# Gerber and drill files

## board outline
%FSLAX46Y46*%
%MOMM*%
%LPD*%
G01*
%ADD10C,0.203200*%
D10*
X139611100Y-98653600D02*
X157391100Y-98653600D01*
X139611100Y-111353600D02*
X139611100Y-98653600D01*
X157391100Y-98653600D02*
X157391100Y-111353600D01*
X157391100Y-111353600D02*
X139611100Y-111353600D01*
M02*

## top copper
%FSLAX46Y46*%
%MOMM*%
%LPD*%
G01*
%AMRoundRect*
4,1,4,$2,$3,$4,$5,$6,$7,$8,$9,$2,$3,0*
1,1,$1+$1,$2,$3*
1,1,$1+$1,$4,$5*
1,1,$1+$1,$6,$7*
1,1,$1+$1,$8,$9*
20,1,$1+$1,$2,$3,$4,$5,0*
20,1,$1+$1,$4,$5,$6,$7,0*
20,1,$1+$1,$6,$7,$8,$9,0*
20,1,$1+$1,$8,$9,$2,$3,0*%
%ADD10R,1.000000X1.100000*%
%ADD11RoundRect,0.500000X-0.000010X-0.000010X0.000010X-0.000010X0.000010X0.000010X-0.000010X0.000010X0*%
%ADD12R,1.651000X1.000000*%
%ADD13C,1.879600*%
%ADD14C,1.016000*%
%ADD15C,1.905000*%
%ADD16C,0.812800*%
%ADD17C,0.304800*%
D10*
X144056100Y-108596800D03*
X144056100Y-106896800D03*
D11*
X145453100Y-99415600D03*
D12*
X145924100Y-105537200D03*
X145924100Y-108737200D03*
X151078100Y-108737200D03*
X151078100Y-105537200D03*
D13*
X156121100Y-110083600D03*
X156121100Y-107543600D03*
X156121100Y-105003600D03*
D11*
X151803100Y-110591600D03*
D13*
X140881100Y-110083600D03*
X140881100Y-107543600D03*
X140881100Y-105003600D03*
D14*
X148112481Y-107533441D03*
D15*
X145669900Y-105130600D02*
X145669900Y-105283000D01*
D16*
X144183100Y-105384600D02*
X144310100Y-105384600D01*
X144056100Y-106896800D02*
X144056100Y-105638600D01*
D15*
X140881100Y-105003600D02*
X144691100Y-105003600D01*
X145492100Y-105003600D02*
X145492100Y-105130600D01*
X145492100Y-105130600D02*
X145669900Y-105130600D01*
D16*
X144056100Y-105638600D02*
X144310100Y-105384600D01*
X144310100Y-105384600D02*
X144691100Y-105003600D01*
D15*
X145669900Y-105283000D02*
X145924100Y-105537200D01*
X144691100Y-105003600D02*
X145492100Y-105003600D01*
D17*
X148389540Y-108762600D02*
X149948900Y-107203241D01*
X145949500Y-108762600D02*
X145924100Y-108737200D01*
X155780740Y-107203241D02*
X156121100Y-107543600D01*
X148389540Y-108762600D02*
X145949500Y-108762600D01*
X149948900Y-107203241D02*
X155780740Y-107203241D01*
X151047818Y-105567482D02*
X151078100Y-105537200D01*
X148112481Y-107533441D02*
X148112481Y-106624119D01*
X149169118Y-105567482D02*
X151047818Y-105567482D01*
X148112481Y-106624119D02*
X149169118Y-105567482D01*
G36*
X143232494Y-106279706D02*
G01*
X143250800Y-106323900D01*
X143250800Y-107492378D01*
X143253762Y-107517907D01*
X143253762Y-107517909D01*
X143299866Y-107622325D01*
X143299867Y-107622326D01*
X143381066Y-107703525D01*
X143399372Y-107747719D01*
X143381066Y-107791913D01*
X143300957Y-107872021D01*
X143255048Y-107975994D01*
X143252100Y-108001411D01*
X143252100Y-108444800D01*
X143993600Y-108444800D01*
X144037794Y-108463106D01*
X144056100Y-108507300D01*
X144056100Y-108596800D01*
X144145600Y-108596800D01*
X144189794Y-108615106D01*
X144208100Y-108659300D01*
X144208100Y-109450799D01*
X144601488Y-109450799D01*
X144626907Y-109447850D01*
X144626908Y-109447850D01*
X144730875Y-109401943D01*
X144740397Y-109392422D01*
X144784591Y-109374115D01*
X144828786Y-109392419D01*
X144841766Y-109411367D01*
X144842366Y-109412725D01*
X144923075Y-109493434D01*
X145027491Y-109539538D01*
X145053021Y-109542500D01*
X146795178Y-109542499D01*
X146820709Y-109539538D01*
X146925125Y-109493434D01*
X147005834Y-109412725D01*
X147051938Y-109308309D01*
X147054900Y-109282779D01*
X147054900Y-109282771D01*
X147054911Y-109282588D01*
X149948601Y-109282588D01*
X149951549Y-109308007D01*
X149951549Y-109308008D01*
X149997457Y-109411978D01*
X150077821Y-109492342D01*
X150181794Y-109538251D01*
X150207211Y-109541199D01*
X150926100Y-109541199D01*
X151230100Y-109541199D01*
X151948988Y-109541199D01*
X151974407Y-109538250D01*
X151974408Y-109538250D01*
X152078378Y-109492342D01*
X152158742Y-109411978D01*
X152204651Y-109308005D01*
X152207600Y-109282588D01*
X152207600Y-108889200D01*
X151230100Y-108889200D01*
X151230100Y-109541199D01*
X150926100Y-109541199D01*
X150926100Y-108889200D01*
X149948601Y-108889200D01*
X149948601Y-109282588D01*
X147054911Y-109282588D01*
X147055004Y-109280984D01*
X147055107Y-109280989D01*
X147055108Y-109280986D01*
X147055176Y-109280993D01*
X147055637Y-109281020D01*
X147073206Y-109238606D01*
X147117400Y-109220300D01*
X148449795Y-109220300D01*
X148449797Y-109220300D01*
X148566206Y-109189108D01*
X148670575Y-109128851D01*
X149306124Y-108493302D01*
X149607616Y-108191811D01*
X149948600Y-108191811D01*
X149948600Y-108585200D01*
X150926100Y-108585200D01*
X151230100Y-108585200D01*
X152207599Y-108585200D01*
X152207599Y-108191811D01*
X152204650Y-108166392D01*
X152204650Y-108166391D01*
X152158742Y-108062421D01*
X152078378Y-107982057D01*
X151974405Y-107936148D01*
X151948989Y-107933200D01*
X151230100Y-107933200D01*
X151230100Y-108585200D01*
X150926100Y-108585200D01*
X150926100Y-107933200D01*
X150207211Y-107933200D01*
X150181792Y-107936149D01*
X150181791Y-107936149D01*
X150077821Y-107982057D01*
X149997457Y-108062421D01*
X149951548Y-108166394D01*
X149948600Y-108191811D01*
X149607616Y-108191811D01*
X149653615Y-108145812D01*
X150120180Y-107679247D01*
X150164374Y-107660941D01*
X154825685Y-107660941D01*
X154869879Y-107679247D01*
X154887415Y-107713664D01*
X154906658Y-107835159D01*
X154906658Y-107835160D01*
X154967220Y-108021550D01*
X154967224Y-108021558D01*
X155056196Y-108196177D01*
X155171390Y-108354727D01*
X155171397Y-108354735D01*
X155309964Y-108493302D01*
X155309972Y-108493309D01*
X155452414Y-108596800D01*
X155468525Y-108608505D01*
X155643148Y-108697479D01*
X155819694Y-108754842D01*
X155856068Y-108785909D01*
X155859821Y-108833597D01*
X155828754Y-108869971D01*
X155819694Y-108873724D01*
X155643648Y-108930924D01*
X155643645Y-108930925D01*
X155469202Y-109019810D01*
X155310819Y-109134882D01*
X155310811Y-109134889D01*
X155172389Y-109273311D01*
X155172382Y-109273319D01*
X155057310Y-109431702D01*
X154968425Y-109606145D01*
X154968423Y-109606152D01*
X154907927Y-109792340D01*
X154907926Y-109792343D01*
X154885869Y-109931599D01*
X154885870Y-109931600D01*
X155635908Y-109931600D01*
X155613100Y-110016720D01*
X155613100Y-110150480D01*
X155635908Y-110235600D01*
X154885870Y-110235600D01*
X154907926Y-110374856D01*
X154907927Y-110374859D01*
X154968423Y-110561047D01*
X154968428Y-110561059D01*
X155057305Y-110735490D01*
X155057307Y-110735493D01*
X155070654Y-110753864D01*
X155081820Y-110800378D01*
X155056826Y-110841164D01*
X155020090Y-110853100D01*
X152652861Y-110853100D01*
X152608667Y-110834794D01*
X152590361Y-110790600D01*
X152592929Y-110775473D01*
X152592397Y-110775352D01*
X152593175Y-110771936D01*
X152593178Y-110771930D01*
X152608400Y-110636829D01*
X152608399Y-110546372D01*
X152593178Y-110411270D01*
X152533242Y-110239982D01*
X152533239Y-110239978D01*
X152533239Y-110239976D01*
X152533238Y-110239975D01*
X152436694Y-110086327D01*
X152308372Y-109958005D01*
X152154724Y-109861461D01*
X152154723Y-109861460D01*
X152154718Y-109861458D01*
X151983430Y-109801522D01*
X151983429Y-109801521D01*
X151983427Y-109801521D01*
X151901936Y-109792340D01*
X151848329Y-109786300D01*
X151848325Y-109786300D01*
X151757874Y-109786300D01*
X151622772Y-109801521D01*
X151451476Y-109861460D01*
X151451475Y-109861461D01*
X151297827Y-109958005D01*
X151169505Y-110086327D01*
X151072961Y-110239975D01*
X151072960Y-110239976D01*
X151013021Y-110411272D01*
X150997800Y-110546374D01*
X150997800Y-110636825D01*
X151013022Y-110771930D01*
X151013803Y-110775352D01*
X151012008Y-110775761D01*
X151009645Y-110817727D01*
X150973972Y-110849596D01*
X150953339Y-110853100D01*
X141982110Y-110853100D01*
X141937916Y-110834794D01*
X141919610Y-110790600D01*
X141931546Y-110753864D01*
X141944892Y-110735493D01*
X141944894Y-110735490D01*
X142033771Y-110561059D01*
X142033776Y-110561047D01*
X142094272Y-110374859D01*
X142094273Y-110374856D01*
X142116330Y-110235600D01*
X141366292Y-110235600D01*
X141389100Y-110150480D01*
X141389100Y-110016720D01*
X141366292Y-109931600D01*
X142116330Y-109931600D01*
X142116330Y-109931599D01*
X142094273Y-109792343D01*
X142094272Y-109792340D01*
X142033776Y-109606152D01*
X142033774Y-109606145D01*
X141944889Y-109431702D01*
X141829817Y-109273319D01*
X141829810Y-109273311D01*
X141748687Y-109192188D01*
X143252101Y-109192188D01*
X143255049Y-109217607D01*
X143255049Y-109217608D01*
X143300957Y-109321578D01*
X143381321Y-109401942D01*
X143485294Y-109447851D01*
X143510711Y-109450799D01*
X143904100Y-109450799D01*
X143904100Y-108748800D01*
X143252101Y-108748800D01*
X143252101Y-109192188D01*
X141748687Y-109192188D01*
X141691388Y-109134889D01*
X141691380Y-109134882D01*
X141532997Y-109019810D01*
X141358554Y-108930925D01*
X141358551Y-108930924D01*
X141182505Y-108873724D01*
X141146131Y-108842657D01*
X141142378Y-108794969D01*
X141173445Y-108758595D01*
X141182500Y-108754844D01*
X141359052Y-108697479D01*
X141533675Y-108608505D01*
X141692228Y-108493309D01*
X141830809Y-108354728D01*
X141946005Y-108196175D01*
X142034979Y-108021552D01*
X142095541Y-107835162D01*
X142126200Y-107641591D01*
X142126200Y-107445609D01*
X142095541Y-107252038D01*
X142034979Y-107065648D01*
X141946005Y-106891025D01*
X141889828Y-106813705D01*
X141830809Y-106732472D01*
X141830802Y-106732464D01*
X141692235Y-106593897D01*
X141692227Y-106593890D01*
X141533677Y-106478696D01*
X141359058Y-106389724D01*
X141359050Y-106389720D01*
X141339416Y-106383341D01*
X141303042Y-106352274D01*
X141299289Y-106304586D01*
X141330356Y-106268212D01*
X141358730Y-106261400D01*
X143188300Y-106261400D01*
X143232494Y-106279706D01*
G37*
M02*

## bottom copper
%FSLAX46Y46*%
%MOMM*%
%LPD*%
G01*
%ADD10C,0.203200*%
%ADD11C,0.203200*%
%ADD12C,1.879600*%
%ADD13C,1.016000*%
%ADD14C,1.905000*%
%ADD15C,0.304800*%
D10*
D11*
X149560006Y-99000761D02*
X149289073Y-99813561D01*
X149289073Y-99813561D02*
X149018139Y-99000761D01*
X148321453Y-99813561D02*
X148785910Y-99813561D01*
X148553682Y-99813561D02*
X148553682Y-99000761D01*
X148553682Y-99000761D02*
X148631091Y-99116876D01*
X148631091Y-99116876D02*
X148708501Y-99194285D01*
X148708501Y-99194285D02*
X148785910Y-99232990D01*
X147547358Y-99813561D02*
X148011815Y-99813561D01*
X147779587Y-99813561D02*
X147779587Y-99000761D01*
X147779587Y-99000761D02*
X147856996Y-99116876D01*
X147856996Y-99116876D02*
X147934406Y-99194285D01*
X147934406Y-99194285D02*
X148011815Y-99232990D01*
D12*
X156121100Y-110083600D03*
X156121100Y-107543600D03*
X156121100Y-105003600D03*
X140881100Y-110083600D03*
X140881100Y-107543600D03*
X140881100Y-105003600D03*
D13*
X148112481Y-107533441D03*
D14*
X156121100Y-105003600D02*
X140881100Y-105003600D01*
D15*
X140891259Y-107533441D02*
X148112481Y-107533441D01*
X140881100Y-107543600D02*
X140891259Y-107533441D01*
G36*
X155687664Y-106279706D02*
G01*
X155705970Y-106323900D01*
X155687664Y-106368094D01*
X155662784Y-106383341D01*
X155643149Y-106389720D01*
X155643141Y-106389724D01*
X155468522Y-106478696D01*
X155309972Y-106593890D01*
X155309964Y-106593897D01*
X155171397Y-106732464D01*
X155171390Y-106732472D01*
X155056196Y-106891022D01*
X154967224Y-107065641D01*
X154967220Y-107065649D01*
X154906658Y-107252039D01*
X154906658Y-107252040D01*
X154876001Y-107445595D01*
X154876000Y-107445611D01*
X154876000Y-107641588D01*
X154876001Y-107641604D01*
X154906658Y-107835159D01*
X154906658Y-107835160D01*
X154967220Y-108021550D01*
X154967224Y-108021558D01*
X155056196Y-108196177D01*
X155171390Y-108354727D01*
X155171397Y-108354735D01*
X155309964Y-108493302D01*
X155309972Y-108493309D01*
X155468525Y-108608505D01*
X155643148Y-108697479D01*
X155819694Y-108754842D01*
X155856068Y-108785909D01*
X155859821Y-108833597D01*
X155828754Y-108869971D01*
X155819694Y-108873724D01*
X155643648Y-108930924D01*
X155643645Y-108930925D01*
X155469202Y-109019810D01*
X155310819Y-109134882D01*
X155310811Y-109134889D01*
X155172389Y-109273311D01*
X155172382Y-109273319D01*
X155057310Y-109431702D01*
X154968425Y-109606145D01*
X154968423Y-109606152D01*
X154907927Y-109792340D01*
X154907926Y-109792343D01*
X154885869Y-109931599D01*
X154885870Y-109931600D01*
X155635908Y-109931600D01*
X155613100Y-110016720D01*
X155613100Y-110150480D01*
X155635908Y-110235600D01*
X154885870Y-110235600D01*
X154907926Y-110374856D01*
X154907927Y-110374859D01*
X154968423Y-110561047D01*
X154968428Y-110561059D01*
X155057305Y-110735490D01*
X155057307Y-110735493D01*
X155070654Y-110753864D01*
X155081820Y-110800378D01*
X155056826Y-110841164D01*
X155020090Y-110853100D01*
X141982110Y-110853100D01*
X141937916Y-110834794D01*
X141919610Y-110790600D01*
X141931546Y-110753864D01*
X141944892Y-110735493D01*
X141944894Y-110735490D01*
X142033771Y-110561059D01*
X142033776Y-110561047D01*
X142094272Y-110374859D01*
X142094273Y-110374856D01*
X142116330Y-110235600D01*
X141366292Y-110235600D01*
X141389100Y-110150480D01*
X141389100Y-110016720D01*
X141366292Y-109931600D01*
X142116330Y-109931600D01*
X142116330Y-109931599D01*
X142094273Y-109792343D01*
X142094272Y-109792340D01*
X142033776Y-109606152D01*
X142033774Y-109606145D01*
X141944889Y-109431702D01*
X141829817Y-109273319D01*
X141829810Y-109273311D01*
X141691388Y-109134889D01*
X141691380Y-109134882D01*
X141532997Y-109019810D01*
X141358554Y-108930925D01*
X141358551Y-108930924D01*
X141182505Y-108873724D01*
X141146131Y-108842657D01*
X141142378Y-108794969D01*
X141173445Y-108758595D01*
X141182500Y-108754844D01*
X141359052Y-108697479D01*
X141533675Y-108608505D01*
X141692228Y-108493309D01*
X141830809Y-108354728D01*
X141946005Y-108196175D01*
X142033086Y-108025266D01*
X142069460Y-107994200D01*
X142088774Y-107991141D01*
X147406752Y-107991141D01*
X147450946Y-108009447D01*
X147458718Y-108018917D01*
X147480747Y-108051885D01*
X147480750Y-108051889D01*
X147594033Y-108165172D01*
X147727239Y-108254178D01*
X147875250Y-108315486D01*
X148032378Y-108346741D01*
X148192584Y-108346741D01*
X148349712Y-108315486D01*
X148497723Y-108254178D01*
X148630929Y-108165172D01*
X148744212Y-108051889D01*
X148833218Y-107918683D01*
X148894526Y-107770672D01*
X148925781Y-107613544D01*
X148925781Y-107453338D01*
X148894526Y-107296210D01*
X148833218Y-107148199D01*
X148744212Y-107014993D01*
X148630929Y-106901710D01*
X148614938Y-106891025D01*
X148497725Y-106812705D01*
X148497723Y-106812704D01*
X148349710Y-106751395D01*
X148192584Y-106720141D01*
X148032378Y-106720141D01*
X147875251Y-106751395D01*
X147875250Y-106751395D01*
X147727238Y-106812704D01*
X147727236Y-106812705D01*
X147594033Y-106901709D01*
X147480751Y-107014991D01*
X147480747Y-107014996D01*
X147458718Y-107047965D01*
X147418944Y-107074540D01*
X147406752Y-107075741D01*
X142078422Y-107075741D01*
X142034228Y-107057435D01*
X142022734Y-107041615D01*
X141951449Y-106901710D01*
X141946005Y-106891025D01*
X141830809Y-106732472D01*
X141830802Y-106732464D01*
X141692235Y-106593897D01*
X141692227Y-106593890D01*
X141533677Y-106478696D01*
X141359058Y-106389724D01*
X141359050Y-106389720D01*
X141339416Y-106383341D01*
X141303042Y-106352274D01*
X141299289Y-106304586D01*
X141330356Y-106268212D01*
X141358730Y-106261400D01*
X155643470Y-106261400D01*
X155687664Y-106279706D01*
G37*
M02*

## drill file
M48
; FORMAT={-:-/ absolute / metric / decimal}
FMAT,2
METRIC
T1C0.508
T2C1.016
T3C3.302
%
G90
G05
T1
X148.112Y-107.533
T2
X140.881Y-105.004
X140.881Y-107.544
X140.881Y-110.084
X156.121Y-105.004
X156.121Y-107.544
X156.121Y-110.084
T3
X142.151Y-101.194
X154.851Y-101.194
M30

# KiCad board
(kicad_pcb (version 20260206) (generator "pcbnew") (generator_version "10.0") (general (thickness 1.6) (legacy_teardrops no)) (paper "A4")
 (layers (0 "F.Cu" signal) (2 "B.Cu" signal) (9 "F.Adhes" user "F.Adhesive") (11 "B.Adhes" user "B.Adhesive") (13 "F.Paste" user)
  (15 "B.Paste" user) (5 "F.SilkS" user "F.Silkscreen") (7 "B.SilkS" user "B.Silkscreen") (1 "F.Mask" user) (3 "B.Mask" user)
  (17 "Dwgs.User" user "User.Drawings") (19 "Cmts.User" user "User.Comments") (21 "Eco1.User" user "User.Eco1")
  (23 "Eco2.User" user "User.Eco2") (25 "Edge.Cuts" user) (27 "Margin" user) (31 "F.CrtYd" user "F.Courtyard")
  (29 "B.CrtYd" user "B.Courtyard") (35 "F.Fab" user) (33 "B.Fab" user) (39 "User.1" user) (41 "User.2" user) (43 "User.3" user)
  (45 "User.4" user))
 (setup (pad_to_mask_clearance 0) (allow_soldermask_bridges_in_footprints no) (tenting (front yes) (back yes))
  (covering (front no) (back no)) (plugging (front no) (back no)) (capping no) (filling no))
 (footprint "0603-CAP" (layer "F.Cu") (at 144.0561 107.7468 90)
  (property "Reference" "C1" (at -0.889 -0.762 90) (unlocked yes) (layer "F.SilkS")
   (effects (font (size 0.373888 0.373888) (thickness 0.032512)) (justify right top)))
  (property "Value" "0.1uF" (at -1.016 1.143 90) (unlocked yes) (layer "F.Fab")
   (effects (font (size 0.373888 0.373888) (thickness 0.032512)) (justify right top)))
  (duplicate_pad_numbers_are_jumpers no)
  (pad "1" smd rect (at -0.85 0 90) (size 1.1 1) (layers "F.Cu" "F.Mask" "F.Paste") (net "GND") (solder_mask_margin 0.1016)
   (solder_paste_margin 0) (thermal_bridge_angle 0))
  (pad "2" smd rect (at 0.85 0 90) (size 1.1 1) (layers "F.Cu" "F.Mask" "F.Paste") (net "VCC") (solder_mask_margin 0.1016)
   (solder_paste_margin 0) (thermal_bridge_angle 0)))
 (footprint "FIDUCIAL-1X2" (layer "F.Cu") (at 145.4531 99.4156)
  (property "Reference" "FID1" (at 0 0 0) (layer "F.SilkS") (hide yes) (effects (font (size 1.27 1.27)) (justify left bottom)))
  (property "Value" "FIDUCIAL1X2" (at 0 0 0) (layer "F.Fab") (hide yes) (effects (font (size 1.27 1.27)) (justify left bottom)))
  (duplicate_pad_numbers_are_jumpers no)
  (pad "1" smd roundrect (at 0 0) (size 1 1) (layers "F.Cu" "F.Mask") (roundrect_rratio 0.5) (solder_mask_margin 0.1016)
   (solder_paste_margin 0) (thermal_bridge_angle 0)))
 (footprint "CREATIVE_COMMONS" (layer "F.Cu") (at 118.159513 124.0536)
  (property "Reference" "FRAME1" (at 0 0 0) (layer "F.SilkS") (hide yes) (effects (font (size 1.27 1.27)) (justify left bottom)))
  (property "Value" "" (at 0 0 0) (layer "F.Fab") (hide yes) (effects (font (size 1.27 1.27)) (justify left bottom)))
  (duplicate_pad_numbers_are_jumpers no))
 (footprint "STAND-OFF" (layer "F.Cu") (at 154.8511 101.1936)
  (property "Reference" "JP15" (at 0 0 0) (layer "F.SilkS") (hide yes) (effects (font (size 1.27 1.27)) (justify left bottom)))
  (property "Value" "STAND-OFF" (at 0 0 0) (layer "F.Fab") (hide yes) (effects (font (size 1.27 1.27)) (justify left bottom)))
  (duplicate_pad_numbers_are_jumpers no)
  (pad "" np_thru_hole circle (at 0 0) (size 3.302 3.302) (drill 3.302) (layers "*.Cu" "*.Mask")))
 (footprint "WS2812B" (layer "F.Cu") (at 148.5011 107.1372)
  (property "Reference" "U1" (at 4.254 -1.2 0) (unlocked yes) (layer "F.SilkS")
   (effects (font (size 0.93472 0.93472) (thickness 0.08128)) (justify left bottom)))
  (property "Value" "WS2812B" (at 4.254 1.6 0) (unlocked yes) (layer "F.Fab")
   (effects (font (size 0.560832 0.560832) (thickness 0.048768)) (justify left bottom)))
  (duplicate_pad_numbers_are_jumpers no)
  (pad "1" smd rect (at -2.577 -1.6) (size 1.651 1) (layers "F.Cu" "F.Mask" "F.Paste") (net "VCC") (solder_mask_margin 0.1016)
   (solder_paste_margin 0) (thermal_bridge_angle 0))
  (pad "2" smd rect (at -2.577 1.6) (size 1.651 1) (layers "F.Cu" "F.Mask" "F.Paste") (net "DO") (solder_mask_margin 0.1016)
   (solder_paste_margin 0) (thermal_bridge_angle 0))
  (pad "3" smd rect (at 2.577 1.6) (size 1.651 1) (layers "F.Cu" "F.Mask" "F.Paste") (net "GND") (solder_mask_margin 0.1016)
   (solder_paste_margin 0) (thermal_bridge_angle 0))
  (pad "4" smd rect (at 2.577 -1.6) (size 1.651 1) (layers "F.Cu" "F.Mask" "F.Paste") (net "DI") (solder_mask_margin 0.1016)
   (solder_paste_margin 0) (thermal_bridge_angle 0)))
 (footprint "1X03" (layer "F.Cu") (at 156.1211 110.0836 90)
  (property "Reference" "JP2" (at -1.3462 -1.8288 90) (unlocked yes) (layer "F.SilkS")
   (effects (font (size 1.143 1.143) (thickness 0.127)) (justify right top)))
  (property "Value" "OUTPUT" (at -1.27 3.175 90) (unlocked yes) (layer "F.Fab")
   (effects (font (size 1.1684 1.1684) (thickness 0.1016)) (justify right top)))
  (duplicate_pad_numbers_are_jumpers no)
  (pad "1" thru_hole circle (at 0 0 180) (size 1.8796 1.8796) (drill 1.016) (layers "*.Cu" "*.Mask") (remove_unused_layers no) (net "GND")
   (solder_mask_margin 0.1016) (thermal_bridge_angle 0))
  (pad "2" thru_hole circle (at 2.54 0 180) (size 1.8796 1.8796) (drill 1.016) (layers "*.Cu" "*.Mask") (remove_unused_layers no) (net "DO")
   (solder_mask_margin 0.1016) (thermal_bridge_angle 0))
  (pad "3" thru_hole circle (at 5.08 0 180) (size 1.8796 1.8796) (drill 1.016) (layers "*.Cu" "*.Mask") (remove_unused_layers no)
   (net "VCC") (solder_mask_margin 0.1016) (thermal_bridge_angle 0)))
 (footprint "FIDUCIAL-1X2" (layer "F.Cu") (at 151.8031 110.5916)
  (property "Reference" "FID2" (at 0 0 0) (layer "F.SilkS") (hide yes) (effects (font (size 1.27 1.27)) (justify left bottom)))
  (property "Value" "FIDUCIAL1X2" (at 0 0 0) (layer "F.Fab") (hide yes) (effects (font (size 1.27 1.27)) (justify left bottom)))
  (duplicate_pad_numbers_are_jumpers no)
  (pad "1" smd roundrect (at 0 0) (size 1 1) (layers "F.Cu" "F.Mask") (roundrect_rratio 0.5) (solder_mask_margin 0.1016)
   (solder_paste_margin 0) (thermal_bridge_angle 0)))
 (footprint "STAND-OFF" (layer "F.Cu") (at 142.1511 101.1936)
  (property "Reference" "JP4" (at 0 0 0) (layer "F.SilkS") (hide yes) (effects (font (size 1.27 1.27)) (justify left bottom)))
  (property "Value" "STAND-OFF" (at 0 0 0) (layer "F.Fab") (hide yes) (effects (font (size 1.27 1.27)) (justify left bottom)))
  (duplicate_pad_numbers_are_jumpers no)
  (pad "" np_thru_hole circle (at 0 0) (size 3.302 3.302) (drill 3.302) (layers "*.Cu" "*.Mask")))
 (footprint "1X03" (layer "F.Cu") (at 140.8811 110.0836 90)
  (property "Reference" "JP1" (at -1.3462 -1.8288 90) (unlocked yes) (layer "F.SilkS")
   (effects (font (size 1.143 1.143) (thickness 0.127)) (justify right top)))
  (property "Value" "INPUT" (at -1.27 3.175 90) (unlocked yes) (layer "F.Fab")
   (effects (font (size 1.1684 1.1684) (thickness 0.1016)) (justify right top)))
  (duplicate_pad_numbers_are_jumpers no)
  (pad "1" thru_hole circle (at 0 0 180) (size 1.8796 1.8796) (drill 1.016) (layers "*.Cu" "*.Mask") (remove_unused_layers no) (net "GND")
   (solder_mask_margin 0.1016) (thermal_bridge_angle 0))
  (pad "2" thru_hole circle (at 2.54 0 180) (size 1.8796 1.8796) (drill 1.016) (layers "*.Cu" "*.Mask") (remove_unused_layers no) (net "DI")
   (solder_mask_margin 0.1016) (thermal_bridge_angle 0))
  (pad "3" thru_hole circle (at 5.08 0 180) (size 1.8796 1.8796) (drill 1.016) (layers "*.Cu" "*.Mask") (remove_unused_layers no)
   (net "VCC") (solder_mask_margin 0.1016) (thermal_bridge_angle 0)))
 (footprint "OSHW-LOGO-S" (layer "B.Cu") (at 148.587459 102.217222 180)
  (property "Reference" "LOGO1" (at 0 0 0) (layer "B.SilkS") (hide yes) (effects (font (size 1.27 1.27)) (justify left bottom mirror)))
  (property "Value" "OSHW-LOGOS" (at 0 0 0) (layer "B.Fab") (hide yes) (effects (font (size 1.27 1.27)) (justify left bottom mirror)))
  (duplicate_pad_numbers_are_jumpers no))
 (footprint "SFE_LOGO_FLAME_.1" (layer "B.Cu") (at 149.768559 106.913679 180)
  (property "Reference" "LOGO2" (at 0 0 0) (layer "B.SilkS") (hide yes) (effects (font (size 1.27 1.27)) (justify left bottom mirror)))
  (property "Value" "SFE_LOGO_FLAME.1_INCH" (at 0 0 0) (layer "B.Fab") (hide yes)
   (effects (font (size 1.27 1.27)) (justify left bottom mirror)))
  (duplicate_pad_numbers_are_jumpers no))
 (gr_line (start 139.6111 98.6536) (end 157.3911 98.6536) (stroke (width 0.2032) (type solid)) (layer "Edge.Cuts"))
 (gr_line (start 139.6111 111.3536) (end 139.6111 98.6536) (stroke (width 0.2032) (type solid)) (layer "Edge.Cuts"))
 (gr_line (start 157.3911 98.6536) (end 157.3911 111.3536) (stroke (width 0.2032) (type solid)) (layer "Edge.Cuts"))
 (gr_line (start 157.3911 111.3536) (end 139.6111 111.3536) (stroke (width 0.2032) (type solid)) (layer "Edge.Cuts"))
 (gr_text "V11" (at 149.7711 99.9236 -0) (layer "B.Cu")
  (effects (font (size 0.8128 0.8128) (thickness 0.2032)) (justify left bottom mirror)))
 (segment (start 145.6699 105.1306) (end 145.6699 105.283) (width 1.905) (layer "F.Cu") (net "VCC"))
 (segment (start 144.1831 105.3846) (end 144.3101 105.3846) (width 0.8128) (layer "F.Cu") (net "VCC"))
 (segment (start 144.0561 106.8968) (end 144.0561 105.6386) (width 0.8128) (layer "F.Cu") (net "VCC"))
 (segment (start 140.8811 105.0036) (end 144.6911 105.0036) (width 1.905) (layer "F.Cu") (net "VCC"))
 (segment (start 145.4921 105.0036) (end 145.4921 105.1306) (width 1.905) (layer "F.Cu") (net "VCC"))
 (segment (start 145.4921 105.1306) (end 145.6699 105.1306) (width 1.905) (layer "F.Cu") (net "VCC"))
 (segment (start 144.0561 105.6386) (end 144.3101 105.3846) (width 0.8128) (layer "F.Cu") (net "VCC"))
 (segment (start 144.3101 105.3846) (end 144.6911 105.0036) (width 0.8128) (layer "F.Cu") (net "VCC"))
 (segment (start 145.6699 105.283) (end 145.9241 105.5372) (width 1.905) (layer "F.Cu") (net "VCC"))
 (segment (start 144.6911 105.0036) (end 145.4921 105.0036) (width 1.905) (layer "F.Cu") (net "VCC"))
 (segment (start 156.1211 105.0036) (end 140.8811 105.0036) (width 1.905) (layer "B.Cu") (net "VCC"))
 (segment (start 148.38954 108.7626) (end 149.9489 107.203241) (width 0.3048) (layer "F.Cu") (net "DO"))
 (segment (start 145.9495 108.7626) (end 145.9241 108.7372) (width 0.3048) (layer "F.Cu") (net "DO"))
 (segment (start 155.78074 107.203241) (end 156.1211 107.5436) (width 0.3048) (layer "F.Cu") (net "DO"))
 (segment (start 148.38954 108.7626) (end 145.9495 108.7626) (width 0.3048) (layer "F.Cu") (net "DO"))
 (segment (start 149.9489 107.203241) (end 155.78074 107.203241) (width 0.3048) (layer "F.Cu") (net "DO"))
 (segment (start 151.047818 105.567482) (end 151.0781 105.5372) (width 0.3048) (layer "F.Cu") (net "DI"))
 (segment (start 148.112481 107.533441) (end 148.112481 106.624119) (width 0.3048) (layer "F.Cu") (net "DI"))
 (segment (start 149.169118 105.567482) (end 151.047818 105.567482) (width 0.3048) (layer "F.Cu") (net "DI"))
 (segment (start 148.112481 106.624119) (end 149.169118 105.567482) (width 0.3048) (layer "F.Cu") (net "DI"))
 (via (at 148.112481 107.533441) (size 1.016) (drill 0.508) (layers "F.Cu" "B.Cu") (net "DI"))
 (segment (start 140.891259 107.533441) (end 148.112481 107.533441) (width 0.3048) (layer "B.Cu") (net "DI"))
 (segment (start 140.8811 107.5436) (end 140.891259 107.533441) (width 0.3048) (layer "B.Cu") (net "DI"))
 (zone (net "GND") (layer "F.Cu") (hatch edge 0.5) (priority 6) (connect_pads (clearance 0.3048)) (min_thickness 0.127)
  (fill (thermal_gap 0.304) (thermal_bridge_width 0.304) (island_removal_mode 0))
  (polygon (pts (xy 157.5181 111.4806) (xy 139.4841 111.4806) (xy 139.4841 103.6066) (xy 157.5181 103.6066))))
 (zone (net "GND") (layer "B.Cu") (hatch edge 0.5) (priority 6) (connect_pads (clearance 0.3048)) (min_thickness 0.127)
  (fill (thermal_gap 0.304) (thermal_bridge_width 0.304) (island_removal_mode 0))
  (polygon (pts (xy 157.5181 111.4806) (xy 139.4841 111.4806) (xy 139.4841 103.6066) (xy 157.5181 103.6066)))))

